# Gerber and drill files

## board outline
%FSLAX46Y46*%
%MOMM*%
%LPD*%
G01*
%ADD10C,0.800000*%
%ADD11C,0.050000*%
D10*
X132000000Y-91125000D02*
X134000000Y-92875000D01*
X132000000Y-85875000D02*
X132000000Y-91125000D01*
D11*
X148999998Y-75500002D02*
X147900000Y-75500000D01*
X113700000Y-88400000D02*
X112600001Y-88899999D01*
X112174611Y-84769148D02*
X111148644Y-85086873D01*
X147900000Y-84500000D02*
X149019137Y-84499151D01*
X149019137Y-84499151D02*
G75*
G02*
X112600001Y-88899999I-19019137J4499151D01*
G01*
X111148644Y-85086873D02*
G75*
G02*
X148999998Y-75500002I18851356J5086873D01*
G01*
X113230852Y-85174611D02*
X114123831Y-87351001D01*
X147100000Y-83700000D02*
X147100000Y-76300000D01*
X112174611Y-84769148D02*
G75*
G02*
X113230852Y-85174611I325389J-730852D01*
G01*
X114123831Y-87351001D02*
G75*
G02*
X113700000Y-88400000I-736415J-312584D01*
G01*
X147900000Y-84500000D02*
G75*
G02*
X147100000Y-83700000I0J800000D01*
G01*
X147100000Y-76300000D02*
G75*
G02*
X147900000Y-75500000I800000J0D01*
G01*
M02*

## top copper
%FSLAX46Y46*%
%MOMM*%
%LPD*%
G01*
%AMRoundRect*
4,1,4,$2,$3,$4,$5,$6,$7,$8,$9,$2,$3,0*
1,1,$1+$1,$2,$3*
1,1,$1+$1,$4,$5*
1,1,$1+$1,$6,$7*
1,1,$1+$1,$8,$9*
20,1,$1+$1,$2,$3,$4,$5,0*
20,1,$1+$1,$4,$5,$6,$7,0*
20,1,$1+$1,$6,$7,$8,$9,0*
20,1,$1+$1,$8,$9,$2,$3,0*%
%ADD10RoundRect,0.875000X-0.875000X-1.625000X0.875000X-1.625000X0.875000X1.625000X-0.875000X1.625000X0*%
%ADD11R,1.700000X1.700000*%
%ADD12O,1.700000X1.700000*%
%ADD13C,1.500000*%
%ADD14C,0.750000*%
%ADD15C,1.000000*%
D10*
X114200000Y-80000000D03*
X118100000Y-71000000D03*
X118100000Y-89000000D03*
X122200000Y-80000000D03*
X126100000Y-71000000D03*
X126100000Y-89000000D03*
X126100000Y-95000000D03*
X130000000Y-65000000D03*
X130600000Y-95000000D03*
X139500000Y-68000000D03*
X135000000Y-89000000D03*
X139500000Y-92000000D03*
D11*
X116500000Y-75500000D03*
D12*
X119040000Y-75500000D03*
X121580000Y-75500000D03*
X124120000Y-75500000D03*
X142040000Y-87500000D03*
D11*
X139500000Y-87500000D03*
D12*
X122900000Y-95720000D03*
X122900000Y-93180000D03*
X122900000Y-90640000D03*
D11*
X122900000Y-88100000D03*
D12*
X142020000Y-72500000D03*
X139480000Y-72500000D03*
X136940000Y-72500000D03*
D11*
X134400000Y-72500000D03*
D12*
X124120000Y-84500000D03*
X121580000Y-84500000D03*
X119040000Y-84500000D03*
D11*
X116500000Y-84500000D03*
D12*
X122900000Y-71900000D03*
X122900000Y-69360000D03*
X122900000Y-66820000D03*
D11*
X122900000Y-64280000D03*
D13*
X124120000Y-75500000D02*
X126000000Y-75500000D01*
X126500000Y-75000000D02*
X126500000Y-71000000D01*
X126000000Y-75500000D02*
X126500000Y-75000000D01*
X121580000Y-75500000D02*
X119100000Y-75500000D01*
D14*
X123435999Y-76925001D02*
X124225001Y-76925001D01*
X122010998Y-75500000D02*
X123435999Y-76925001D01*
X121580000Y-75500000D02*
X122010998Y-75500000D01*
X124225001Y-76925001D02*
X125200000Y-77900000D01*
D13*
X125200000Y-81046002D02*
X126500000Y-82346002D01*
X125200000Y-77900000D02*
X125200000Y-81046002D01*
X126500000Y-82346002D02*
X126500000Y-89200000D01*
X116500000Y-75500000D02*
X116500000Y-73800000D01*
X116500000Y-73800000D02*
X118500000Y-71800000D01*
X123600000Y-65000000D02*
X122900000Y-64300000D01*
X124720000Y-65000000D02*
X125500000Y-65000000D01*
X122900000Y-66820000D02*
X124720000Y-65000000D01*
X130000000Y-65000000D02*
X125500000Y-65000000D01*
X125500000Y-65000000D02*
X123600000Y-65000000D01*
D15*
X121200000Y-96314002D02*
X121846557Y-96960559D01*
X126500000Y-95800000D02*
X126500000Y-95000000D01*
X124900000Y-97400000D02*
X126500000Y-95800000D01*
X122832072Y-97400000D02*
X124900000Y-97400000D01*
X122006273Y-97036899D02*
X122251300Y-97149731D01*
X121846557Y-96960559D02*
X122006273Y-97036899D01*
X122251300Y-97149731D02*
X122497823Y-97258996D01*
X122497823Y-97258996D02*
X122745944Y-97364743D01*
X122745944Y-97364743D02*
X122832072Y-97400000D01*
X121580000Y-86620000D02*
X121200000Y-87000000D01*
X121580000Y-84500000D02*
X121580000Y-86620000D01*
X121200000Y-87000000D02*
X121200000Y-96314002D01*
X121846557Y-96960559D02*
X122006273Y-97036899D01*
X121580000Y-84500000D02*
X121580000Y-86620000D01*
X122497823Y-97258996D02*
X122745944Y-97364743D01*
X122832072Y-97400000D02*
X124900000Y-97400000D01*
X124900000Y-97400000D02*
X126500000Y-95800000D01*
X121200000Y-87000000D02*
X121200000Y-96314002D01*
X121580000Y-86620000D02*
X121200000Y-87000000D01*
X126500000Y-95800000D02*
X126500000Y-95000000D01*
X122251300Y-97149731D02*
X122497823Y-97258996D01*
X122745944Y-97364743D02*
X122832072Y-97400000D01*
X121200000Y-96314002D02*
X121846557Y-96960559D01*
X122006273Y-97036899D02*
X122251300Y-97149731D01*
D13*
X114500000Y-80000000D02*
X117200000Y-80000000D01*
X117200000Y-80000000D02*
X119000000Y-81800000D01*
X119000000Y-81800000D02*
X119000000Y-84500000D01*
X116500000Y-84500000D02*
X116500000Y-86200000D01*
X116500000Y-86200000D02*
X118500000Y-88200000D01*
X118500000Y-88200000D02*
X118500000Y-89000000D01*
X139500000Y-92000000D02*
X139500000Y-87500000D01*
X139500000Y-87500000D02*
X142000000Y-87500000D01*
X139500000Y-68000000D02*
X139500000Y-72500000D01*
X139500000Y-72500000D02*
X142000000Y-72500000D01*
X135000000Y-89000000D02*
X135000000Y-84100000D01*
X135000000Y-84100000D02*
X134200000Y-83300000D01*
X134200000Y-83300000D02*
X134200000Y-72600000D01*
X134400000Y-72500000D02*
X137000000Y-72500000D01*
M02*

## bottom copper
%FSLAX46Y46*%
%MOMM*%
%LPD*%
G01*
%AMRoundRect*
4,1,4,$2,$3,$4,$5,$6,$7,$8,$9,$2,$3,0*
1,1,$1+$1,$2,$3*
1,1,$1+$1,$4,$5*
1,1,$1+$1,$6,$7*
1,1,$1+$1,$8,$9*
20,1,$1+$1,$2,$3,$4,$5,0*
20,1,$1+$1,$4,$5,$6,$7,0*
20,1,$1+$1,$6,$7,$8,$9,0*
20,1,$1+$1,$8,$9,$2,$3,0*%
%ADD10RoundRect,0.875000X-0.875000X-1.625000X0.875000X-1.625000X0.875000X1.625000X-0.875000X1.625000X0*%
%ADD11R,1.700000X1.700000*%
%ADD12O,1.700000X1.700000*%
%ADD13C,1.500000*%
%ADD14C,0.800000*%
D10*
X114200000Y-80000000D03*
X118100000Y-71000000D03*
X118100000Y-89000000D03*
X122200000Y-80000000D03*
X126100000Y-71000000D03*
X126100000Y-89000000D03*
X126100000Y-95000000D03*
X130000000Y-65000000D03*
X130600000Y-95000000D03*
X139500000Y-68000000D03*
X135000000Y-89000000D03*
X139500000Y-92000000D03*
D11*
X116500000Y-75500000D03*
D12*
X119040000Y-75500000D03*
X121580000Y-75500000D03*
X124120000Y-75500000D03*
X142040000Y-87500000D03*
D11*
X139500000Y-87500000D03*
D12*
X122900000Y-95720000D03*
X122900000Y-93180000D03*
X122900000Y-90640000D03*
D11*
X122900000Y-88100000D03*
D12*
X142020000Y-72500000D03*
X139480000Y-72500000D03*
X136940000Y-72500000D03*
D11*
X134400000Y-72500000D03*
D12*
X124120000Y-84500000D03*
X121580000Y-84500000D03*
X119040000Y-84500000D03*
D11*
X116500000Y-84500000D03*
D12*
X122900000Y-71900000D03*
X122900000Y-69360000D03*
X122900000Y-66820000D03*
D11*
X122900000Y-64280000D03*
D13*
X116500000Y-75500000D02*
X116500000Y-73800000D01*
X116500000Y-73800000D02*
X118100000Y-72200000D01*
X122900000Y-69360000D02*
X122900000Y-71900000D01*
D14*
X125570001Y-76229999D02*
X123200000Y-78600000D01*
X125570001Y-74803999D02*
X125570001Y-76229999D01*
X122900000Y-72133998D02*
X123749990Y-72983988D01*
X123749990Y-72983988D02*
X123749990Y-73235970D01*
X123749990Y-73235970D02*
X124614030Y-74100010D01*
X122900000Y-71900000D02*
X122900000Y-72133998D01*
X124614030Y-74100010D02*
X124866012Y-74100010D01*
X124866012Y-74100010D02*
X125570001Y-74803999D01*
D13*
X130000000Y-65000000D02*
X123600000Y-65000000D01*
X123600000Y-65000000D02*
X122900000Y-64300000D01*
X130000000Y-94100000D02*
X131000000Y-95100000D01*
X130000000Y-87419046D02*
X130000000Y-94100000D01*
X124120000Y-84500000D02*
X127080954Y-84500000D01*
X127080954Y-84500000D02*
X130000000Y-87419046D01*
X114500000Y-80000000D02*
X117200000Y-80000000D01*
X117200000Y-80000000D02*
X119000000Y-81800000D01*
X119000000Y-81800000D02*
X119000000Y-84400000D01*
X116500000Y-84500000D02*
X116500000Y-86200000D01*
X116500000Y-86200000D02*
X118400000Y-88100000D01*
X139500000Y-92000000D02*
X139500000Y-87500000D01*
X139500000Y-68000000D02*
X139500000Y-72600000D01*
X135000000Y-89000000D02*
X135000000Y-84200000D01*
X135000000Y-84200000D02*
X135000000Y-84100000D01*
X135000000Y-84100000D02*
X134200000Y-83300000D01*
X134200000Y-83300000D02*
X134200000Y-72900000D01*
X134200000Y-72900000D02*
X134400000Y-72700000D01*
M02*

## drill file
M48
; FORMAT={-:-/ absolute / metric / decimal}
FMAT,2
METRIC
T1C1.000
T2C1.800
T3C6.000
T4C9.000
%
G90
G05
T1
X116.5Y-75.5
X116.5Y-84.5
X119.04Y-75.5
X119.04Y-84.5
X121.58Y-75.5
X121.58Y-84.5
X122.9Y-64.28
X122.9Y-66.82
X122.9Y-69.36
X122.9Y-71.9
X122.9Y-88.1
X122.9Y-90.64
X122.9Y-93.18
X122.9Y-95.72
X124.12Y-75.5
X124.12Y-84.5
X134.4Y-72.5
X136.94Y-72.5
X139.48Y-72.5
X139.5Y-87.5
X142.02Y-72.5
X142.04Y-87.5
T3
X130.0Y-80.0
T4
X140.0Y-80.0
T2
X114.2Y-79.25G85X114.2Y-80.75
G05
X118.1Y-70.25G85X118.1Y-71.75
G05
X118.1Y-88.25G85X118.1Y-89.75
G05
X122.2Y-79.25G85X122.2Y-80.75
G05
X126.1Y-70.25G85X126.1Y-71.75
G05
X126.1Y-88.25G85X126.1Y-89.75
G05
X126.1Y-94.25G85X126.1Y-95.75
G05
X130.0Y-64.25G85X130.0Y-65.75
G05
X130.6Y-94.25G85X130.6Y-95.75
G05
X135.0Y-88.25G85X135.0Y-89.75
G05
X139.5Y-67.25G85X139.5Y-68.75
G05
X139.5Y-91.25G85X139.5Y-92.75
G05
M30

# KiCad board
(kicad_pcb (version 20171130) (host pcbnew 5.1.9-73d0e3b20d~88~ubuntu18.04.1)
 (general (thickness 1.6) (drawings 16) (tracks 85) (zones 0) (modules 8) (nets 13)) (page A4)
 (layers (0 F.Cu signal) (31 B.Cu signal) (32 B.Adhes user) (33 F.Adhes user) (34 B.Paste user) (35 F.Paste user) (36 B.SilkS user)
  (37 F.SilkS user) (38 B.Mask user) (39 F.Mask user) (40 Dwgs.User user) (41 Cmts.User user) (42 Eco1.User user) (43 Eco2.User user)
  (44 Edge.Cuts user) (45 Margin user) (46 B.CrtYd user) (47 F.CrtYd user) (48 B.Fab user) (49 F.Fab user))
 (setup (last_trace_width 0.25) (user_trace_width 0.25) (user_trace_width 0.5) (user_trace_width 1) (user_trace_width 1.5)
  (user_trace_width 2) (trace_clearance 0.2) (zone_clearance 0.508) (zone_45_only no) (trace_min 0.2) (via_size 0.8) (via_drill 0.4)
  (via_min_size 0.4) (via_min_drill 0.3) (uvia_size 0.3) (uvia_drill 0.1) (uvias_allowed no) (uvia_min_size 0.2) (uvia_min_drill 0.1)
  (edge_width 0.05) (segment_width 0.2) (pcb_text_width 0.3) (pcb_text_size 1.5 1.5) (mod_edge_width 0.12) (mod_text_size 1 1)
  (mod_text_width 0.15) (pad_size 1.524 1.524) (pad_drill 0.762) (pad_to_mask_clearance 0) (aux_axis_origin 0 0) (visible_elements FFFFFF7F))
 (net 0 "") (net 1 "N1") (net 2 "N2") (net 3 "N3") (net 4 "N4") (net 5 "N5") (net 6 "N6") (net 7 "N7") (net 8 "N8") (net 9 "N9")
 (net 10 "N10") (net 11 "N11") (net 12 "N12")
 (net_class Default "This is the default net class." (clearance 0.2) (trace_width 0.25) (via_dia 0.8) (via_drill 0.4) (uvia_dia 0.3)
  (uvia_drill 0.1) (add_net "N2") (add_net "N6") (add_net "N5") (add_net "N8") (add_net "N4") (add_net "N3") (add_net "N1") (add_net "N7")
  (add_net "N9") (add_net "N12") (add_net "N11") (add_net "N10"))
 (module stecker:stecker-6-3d (layer F.Cu) (at 130 80)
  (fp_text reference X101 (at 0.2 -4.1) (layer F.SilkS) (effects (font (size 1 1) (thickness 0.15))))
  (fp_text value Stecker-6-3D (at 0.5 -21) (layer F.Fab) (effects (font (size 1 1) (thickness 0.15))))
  (pad "" np_thru_hole circle (at 0 0) (size 6 6) (drill 6) (layers *.Cu *.Mask))
  (pad "" np_thru_hole circle (at 10 0) (size 9 9) (drill 9) (layers *.Cu *.Mask))
  (pad 1 thru_hole roundrect (at -15.8 0) (size 3.5 5) (drill oval 1.8 3.3) (layers *.Cu *.Mask) (roundrect_rratio 0.25) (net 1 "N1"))
  (pad 2 thru_hole roundrect (at -11.9 -9) (size 3.5 5) (drill oval 1.8 3.3) (layers *.Cu *.Mask) (roundrect_rratio 0.25) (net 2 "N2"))
  (pad 5 thru_hole roundrect (at -11.9 9) (size 3.5 5) (drill oval 1.8 3.3) (layers *.Cu *.Mask) (roundrect_rratio 0.25) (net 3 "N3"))
  (pad 8 thru_hole roundrect (at -7.8 0) (size 3.5 5) (drill oval 1.8 3.3) (layers *.Cu *.Mask) (roundrect_rratio 0.25) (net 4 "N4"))
  (pad 12 thru_hole roundrect (at -3.9 -9) (size 3.5 5) (drill oval 1.8 3.3) (layers *.Cu *.Mask) (roundrect_rratio 0.25) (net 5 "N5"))
  (pad 13 thru_hole roundrect (at -3.9 9) (size 3.5 5) (drill oval 1.8 3.3) (layers *.Cu *.Mask) (roundrect_rratio 0.25) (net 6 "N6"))
  (pad 14 thru_hole roundrect (at -3.9 15) (size 3.5 5) (drill oval 1.8 3.3) (layers *.Cu *.Mask) (roundrect_rratio 0.25) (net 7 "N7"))
  (pad 15 thru_hole roundrect (at 0 -15) (size 3.5 5) (drill oval 1.8 3.3) (layers *.Cu *.Mask) (roundrect_rratio 0.25) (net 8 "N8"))
  (pad 18 thru_hole roundrect (at 0.6 15) (size 3.5 5) (drill oval 1.8 3.3) (layers *.Cu *.Mask) (roundrect_rratio 0.25) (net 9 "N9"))
  (pad 23 thru_hole roundrect (at 9.5 -12) (size 3.5 5) (drill oval 1.8 3.3) (layers *.Cu *.Mask) (roundrect_rratio 0.25) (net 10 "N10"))
  (pad 21 thru_hole roundrect (at 5 9) (size 3.5 5) (drill oval 1.8 3.3) (layers *.Cu *.Mask) (roundrect_rratio 0.25) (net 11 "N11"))
  (pad 24 thru_hole roundrect (at 9.5 12) (size 3.5 5) (drill oval 1.8 3.3) (layers *.Cu *.Mask) (roundrect_rratio 0.25) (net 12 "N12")))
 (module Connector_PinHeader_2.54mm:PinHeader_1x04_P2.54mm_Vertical (layer F.Cu) (at 116.5 75.5 90)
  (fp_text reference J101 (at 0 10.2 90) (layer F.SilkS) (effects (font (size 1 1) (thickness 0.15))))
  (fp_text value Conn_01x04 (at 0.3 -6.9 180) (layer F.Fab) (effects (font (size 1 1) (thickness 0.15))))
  (pad 1 thru_hole rect (at 0 0 90) (size 1.7 1.7) (drill 1) (layers *.Cu *.Mask) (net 2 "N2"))
  (pad 2 thru_hole oval (at 0 2.54 90) (size 1.7 1.7) (drill 1) (layers *.Cu *.Mask) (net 6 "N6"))
  (pad 3 thru_hole oval (at 0 5.08 90) (size 1.7 1.7) (drill 1) (layers *.Cu *.Mask) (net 6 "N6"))
  (pad 4 thru_hole oval (at 0 7.62 90) (size 1.7 1.7) (drill 1) (layers *.Cu *.Mask) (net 5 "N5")))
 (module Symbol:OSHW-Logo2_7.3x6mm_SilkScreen (layer F.Cu) (at 134.8 66.7 90)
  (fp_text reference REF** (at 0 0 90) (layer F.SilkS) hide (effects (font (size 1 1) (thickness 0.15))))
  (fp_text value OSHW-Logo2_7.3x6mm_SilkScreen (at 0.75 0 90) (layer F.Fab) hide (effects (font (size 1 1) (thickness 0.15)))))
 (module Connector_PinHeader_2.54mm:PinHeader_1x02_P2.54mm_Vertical (layer F.Cu) (at 139.5 87.5 90)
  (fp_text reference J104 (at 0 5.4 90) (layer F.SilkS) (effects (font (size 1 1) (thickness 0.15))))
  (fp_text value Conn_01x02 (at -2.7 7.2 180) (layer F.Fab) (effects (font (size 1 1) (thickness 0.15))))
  (pad 2 thru_hole oval (at 0 2.54 90) (size 1.7 1.7) (drill 1) (layers *.Cu *.Mask) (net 12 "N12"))
  (pad 1 thru_hole rect (at 0 0 90) (size 1.7 1.7) (drill 1) (layers *.Cu *.Mask) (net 12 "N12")))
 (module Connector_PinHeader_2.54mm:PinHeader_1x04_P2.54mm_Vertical (layer F.Cu) (at 122.9 88.1)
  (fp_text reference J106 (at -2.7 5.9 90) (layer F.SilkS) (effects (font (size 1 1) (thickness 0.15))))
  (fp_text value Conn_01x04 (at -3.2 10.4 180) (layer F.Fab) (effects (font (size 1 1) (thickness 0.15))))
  (pad 4 thru_hole oval (at 0 7.62) (size 1.7 1.7) (drill 1) (layers *.Cu *.Mask))
  (pad 3 thru_hole oval (at 0 5.08) (size 1.7 1.7) (drill 1) (layers *.Cu *.Mask))
  (pad 2 thru_hole oval (at 0 2.54) (size 1.7 1.7) (drill 1) (layers *.Cu *.Mask))
  (pad 1 thru_hole rect (at 0 0) (size 1.7 1.7) (drill 1) (layers *.Cu *.Mask)))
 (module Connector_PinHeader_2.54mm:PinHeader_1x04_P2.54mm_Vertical (layer F.Cu) (at 134.4 72.5 90)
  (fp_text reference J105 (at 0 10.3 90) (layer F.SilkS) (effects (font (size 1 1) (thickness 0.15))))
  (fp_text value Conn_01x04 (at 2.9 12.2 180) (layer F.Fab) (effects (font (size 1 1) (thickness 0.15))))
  (pad 4 thru_hole oval (at 0 7.62 90) (size 1.7 1.7) (drill 1) (layers *.Cu *.Mask) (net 10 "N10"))
  (pad 3 thru_hole oval (at 0 5.08 90) (size 1.7 1.7) (drill 1) (layers *.Cu *.Mask) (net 10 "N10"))
  (pad 2 thru_hole oval (at 0 2.54 90) (size 1.7 1.7) (drill 1) (layers *.Cu *.Mask) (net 11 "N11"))
  (pad 1 thru_hole rect (at 0 0 90) (size 1.7 1.7) (drill 1) (layers *.Cu *.Mask) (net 11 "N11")))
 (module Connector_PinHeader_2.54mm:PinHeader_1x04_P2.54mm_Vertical (layer F.Cu) (at 116.5 84.5 90)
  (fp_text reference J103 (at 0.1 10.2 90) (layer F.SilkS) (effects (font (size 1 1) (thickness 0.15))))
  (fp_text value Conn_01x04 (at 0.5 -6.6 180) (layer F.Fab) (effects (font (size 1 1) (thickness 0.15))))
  (pad 4 thru_hole oval (at 0 7.62 90) (size 1.7 1.7) (drill 1) (layers *.Cu *.Mask) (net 9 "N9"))
  (pad 3 thru_hole oval (at 0 5.08 90) (size 1.7 1.7) (drill 1) (layers *.Cu *.Mask) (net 7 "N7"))
  (pad 2 thru_hole oval (at 0 2.54 90) (size 1.7 1.7) (drill 1) (layers *.Cu *.Mask) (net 1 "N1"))
  (pad 1 thru_hole rect (at 0 0 90) (size 1.7 1.7) (drill 1) (layers *.Cu *.Mask) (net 3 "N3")))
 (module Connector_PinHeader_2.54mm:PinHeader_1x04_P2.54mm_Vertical (layer F.Cu) (at 122.9 64.28)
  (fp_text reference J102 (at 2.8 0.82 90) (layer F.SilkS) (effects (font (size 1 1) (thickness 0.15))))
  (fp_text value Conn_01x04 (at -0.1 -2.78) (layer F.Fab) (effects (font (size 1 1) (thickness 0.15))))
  (pad 4 thru_hole oval (at 0 7.62) (size 1.7 1.7) (drill 1) (layers *.Cu *.Mask) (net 4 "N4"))
  (pad 3 thru_hole oval (at 0 5.08) (size 1.7 1.7) (drill 1) (layers *.Cu *.Mask) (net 4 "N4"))
  (pad 2 thru_hole oval (at 0 2.54) (size 1.7 1.7) (drill 1) (layers *.Cu *.Mask) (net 8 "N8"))
  (pad 1 thru_hole rect (at 0 0) (size 1.7 1.7) (drill 1) (layers *.Cu *.Mask) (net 8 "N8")))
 (gr_line (start 132 91.125) (end 134 92.875) (layer Edge.Cuts) (width 0.8))
 (gr_line (start 132 85.875) (end 132 91.125) (layer Edge.Cuts) (width 0.8))
 (gr_line (start 148.999998 75.500002) (end 147.9 75.5) (layer Edge.Cuts) (width 0.05))
 (gr_line (start 113.7 88.4) (end 112.600001 88.899999) (layer Edge.Cuts) (width 0.05))
 (gr_line (start 112.174611 84.769148) (end 111.148644 85.086873) (layer Edge.Cuts) (width 0.05))
 (gr_line (start 147.9 84.5) (end 149.019137 84.499151) (layer Edge.Cuts) (width 0.05))
 (gr_arc (start 130 80) (end 112.600001 88.899999) (angle -139.6013383) (layer Edge.Cuts) (width 0.05))
 (gr_arc (start 130 80) (end 148.999998 75.500002) (angle -181.7765691) (layer Edge.Cuts) (width 0.05))
 (gr_line (start 113.230852 85.174611) (end 114.123831 87.351001) (layer Edge.Cuts) (width 0.05))
 (gr_line (start 147.1 83.7) (end 147.1 76.3) (layer Edge.Cuts) (width 0.05))
 (gr_arc (start 112.5 85.5) (end 113.230852 85.174611) (angle -90) (layer Edge.Cuts) (width 0.05))
 (gr_arc (start 113.387416 87.663585) (end 113.7 88.4) (angle -90) (layer Edge.Cuts) (width 0.05))
 (gr_arc (start 147.9 83.7) (end 147.1 83.7) (angle -90) (layer Edge.Cuts) (width 0.05))
 (gr_arc (start 147.9 76.3) (end 147.9 75.5) (angle -90) (layer Edge.Cuts) (width 0.05))
 (segment (start 124.12 75.5) (end 126 75.5) (width 1.5) (layer F.Cu) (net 5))
 (segment (start 126.5 75) (end 126.5 71) (width 1.5) (layer F.Cu) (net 5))
 (segment (start 126 75.5) (end 126.5 75) (width 1.5) (layer F.Cu) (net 5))
 (segment (start 121.58 75.5) (end 119.1 75.5) (width 1.5) (layer F.Cu) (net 6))
 (segment (start 123.435999 76.925001) (end 124.225001 76.925001) (width 0.75) (layer F.Cu) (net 6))
 (segment (start 122.010998 75.5) (end 123.435999 76.925001) (width 0.75) (layer F.Cu) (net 6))
 (segment (start 121.58 75.5) (end 122.010998 75.5) (width 0.75) (layer F.Cu) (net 6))
 (segment (start 124.225001 76.925001) (end 125.2 77.9) (width 0.75) (layer F.Cu) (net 6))
 (segment (start 125.2 81.046002) (end 126.5 82.346002) (width 1.5) (layer F.Cu) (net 6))
 (segment (start 125.2 77.9) (end 125.2 81.046002) (width 1.5) (layer F.Cu) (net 6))
 (segment (start 126.5 82.346002) (end 126.5 89.2) (width 1.5) (layer F.Cu) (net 6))
 (segment (start 116.5 75.5) (end 116.5 73.8) (width 1.5) (layer F.Cu) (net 2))
 (segment (start 116.5 73.8) (end 118.5 71.8) (width 1.5) (layer F.Cu) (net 2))
 (segment (start 116.5 75.5) (end 116.5 73.8) (width 1.5) (layer B.Cu) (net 2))
 (segment (start 116.5 73.8) (end 118.1 72.2) (width 1.5) (layer B.Cu) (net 2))
 (segment (start 122.9 69.36) (end 122.9 71.9) (width 1.5) (layer B.Cu) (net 4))
 (segment (start 125.570001 76.229999) (end 123.2 78.6) (width 0.8) (layer B.Cu) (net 4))
 (segment (start 125.570001 74.803999) (end 125.570001 76.229999) (width 0.8) (layer B.Cu) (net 4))
 (segment (start 122.9 72.133998) (end 123.74999 72.983988) (width 0.8) (layer B.Cu) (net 4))
 (segment (start 123.74999 72.983988) (end 123.74999 73.23597) (width 0.8) (layer B.Cu) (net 4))
 (segment (start 123.74999 73.23597) (end 124.61403 74.10001) (width 0.8) (layer B.Cu) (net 4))
 (segment (start 122.9 71.9) (end 122.9 72.133998) (width 0.8) (layer B.Cu) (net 4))
 (segment (start 124.61403 74.10001) (end 124.866012 74.10001) (width 0.8) (layer B.Cu) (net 4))
 (segment (start 124.866012 74.10001) (end 125.570001 74.803999) (width 0.8) (layer B.Cu) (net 4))
 (segment (start 123.6 65) (end 122.9 64.3) (width 1.5) (layer F.Cu) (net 8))
 (segment (start 124.72 65) (end 125.5 65) (width 1.5) (layer F.Cu) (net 8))
 (segment (start 122.9 66.82) (end 124.72 65) (width 1.5) (layer F.Cu) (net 8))
 (segment (start 130 65) (end 125.5 65) (width 1.5) (layer F.Cu) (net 8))
 (segment (start 125.5 65) (end 123.6 65) (width 1.5) (layer F.Cu) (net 8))
 (segment (start 130 65) (end 123.6 65) (width 1.5) (layer B.Cu) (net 8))
 (segment (start 123.6 65) (end 122.9 64.3) (width 1.5) (layer B.Cu) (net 8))
 (segment (start 130 94.1) (end 131 95.1) (width 1.5) (layer B.Cu) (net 9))
 (segment (start 130 87.419046) (end 130 94.1) (width 1.5) (layer B.Cu) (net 9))
 (segment (start 124.12 84.5) (end 127.080954 84.5) (width 1.5) (layer B.Cu) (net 9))
 (segment (start 127.080954 84.5) (end 130 87.419046) (width 1.5) (layer B.Cu) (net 9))
 (segment (start 121.2 96.314002) (end 121.846557 96.960559) (width 1) (layer F.Cu) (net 7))
 (segment (start 126.5 95.8) (end 126.5 95) (width 1) (layer F.Cu) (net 7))
 (segment (start 124.9 97.4) (end 126.5 95.8) (width 1) (layer F.Cu) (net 7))
 (segment (start 122.832072 97.4) (end 124.9 97.4) (width 1) (layer F.Cu) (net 7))
 (segment (start 122.006273 97.036899) (end 122.2513 97.149731) (width 1) (layer F.Cu) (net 7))
 (segment (start 121.846557 96.960559) (end 122.006273 97.036899) (width 1) (layer F.Cu) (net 7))
 (segment (start 122.2513 97.149731) (end 122.497823 97.258996) (width 1) (layer F.Cu) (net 7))
 (segment (start 122.497823 97.258996) (end 122.745944 97.364743) (width 1) (layer F.Cu) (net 7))
 (segment (start 122.745944 97.364743) (end 122.832072 97.4) (width 1) (layer F.Cu) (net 7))
 (segment (start 121.58 86.62) (end 121.2 87) (width 1) (layer F.Cu) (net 7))
 (segment (start 121.58 84.5) (end 121.58 86.62) (width 1) (layer F.Cu) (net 7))
 (segment (start 121.2 87) (end 121.2 96.314002) (width 1) (layer F.Cu) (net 7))
 (segment (start 121.846557 96.960559) (end 122.006273 97.036899) (width 1) (layer F.Cu) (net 7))
 (segment (start 121.58 84.5) (end 121.58 86.62) (width 1) (layer F.Cu) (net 7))
 (segment (start 122.497823 97.258996) (end 122.745944 97.364743) (width 1) (layer F.Cu) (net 7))
 (segment (start 122.832072 97.4) (end 124.9 97.4) (width 1) (layer F.Cu) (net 7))
 (segment (start 124.9 97.4) (end 126.5 95.8) (width 1) (layer F.Cu) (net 7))
 (segment (start 121.2 87) (end 121.2 96.314002) (width 1) (layer F.Cu) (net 7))
 (segment (start 121.58 86.62) (end 121.2 87) (width 1) (layer F.Cu) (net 7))
 (segment (start 126.5 95.8) (end 126.5 95) (width 1) (layer F.Cu) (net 7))
 (segment (start 122.2513 97.149731) (end 122.497823 97.258996) (width 1) (layer F.Cu) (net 7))
 (segment (start 122.745944 97.364743) (end 122.832072 97.4) (width 1) (layer F.Cu) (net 7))
 (segment (start 121.2 96.314002) (end 121.846557 96.960559) (width 1) (layer F.Cu) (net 7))
 (segment (start 122.006273 97.036899) (end 122.2513 97.149731) (width 1) (layer F.Cu) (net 7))
 (segment (start 114.5 80) (end 117.2 80) (width 1.5) (layer F.Cu) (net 1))
 (segment (start 117.2 80) (end 119 81.8) (width 1.5) (layer F.Cu) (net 1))
 (segment (start 119 81.8) (end 119 84.5) (width 1.5) (layer F.Cu) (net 1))
 (segment (start 114.5 80) (end 117.2 80) (width 1.5) (layer B.Cu) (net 1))
 (segment (start 117.2 80) (end 119 81.8) (width 1.5) (layer B.Cu) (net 1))
 (segment (start 119 81.8) (end 119 84.4) (width 1.5) (layer B.Cu) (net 1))
 (segment (start 116.5 84.5) (end 116.5 86.2) (width 1.5) (layer F.Cu) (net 3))
 (segment (start 116.5 86.2) (end 118.5 88.2) (width 1.5) (layer F.Cu) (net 3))
 (segment (start 118.5 88.2) (end 118.5 89) (width 1.5) (layer F.Cu) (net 3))
 (segment (start 116.5 84.5) (end 116.5 86.2) (width 1.5) (layer B.Cu) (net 3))
 (segment (start 116.5 86.2) (end 118.4 88.1) (width 1.5) (layer B.Cu) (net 3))
 (segment (start 139.5 92) (end 139.5 87.5) (width 1.5) (layer F.Cu) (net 12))
 (segment (start 139.5 87.5) (end 142 87.5) (width 1.5) (layer F.Cu) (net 12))
 (segment (start 139.5 92) (end 139.5 87.5) (width 1.5) (layer B.Cu) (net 12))
 (segment (start 139.5 68) (end 139.5 72.5) (width 1.5) (layer F.Cu) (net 10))
 (segment (start 139.5 72.5) (end 142 72.5) (width 1.5) (layer F.Cu) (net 10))
 (segment (start 139.5 68) (end 139.5 72.6) (width 1.5) (layer B.Cu) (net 10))
 (segment (start 135 89) (end 135 84.1) (width 1.5) (layer F.Cu) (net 11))
 (segment (start 135 84.1) (end 134.2 83.3) (width 1.5) (layer F.Cu) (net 11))
 (segment (start 134.2 83.3) (end 134.2 72.6) (width 1.5) (layer F.Cu) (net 11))
 (segment (start 134.4 72.5) (end 137 72.5) (width 1.5) (layer F.Cu) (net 11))
 (segment (start 135 89) (end 135 84.2) (width 1.5) (layer B.Cu) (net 11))
 (segment (start 135 84.2) (end 135 84.1) (width 1.5) (layer B.Cu) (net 11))
 (segment (start 135 84.1) (end 134.2 83.3) (width 1.5) (layer B.Cu) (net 11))
 (segment (start 134.2 83.3) (end 134.2 72.9) (width 1.5) (layer B.Cu) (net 11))
 (segment (start 134.2 72.9) (end 134.4 72.7) (width 1.5) (layer B.Cu) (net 11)))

